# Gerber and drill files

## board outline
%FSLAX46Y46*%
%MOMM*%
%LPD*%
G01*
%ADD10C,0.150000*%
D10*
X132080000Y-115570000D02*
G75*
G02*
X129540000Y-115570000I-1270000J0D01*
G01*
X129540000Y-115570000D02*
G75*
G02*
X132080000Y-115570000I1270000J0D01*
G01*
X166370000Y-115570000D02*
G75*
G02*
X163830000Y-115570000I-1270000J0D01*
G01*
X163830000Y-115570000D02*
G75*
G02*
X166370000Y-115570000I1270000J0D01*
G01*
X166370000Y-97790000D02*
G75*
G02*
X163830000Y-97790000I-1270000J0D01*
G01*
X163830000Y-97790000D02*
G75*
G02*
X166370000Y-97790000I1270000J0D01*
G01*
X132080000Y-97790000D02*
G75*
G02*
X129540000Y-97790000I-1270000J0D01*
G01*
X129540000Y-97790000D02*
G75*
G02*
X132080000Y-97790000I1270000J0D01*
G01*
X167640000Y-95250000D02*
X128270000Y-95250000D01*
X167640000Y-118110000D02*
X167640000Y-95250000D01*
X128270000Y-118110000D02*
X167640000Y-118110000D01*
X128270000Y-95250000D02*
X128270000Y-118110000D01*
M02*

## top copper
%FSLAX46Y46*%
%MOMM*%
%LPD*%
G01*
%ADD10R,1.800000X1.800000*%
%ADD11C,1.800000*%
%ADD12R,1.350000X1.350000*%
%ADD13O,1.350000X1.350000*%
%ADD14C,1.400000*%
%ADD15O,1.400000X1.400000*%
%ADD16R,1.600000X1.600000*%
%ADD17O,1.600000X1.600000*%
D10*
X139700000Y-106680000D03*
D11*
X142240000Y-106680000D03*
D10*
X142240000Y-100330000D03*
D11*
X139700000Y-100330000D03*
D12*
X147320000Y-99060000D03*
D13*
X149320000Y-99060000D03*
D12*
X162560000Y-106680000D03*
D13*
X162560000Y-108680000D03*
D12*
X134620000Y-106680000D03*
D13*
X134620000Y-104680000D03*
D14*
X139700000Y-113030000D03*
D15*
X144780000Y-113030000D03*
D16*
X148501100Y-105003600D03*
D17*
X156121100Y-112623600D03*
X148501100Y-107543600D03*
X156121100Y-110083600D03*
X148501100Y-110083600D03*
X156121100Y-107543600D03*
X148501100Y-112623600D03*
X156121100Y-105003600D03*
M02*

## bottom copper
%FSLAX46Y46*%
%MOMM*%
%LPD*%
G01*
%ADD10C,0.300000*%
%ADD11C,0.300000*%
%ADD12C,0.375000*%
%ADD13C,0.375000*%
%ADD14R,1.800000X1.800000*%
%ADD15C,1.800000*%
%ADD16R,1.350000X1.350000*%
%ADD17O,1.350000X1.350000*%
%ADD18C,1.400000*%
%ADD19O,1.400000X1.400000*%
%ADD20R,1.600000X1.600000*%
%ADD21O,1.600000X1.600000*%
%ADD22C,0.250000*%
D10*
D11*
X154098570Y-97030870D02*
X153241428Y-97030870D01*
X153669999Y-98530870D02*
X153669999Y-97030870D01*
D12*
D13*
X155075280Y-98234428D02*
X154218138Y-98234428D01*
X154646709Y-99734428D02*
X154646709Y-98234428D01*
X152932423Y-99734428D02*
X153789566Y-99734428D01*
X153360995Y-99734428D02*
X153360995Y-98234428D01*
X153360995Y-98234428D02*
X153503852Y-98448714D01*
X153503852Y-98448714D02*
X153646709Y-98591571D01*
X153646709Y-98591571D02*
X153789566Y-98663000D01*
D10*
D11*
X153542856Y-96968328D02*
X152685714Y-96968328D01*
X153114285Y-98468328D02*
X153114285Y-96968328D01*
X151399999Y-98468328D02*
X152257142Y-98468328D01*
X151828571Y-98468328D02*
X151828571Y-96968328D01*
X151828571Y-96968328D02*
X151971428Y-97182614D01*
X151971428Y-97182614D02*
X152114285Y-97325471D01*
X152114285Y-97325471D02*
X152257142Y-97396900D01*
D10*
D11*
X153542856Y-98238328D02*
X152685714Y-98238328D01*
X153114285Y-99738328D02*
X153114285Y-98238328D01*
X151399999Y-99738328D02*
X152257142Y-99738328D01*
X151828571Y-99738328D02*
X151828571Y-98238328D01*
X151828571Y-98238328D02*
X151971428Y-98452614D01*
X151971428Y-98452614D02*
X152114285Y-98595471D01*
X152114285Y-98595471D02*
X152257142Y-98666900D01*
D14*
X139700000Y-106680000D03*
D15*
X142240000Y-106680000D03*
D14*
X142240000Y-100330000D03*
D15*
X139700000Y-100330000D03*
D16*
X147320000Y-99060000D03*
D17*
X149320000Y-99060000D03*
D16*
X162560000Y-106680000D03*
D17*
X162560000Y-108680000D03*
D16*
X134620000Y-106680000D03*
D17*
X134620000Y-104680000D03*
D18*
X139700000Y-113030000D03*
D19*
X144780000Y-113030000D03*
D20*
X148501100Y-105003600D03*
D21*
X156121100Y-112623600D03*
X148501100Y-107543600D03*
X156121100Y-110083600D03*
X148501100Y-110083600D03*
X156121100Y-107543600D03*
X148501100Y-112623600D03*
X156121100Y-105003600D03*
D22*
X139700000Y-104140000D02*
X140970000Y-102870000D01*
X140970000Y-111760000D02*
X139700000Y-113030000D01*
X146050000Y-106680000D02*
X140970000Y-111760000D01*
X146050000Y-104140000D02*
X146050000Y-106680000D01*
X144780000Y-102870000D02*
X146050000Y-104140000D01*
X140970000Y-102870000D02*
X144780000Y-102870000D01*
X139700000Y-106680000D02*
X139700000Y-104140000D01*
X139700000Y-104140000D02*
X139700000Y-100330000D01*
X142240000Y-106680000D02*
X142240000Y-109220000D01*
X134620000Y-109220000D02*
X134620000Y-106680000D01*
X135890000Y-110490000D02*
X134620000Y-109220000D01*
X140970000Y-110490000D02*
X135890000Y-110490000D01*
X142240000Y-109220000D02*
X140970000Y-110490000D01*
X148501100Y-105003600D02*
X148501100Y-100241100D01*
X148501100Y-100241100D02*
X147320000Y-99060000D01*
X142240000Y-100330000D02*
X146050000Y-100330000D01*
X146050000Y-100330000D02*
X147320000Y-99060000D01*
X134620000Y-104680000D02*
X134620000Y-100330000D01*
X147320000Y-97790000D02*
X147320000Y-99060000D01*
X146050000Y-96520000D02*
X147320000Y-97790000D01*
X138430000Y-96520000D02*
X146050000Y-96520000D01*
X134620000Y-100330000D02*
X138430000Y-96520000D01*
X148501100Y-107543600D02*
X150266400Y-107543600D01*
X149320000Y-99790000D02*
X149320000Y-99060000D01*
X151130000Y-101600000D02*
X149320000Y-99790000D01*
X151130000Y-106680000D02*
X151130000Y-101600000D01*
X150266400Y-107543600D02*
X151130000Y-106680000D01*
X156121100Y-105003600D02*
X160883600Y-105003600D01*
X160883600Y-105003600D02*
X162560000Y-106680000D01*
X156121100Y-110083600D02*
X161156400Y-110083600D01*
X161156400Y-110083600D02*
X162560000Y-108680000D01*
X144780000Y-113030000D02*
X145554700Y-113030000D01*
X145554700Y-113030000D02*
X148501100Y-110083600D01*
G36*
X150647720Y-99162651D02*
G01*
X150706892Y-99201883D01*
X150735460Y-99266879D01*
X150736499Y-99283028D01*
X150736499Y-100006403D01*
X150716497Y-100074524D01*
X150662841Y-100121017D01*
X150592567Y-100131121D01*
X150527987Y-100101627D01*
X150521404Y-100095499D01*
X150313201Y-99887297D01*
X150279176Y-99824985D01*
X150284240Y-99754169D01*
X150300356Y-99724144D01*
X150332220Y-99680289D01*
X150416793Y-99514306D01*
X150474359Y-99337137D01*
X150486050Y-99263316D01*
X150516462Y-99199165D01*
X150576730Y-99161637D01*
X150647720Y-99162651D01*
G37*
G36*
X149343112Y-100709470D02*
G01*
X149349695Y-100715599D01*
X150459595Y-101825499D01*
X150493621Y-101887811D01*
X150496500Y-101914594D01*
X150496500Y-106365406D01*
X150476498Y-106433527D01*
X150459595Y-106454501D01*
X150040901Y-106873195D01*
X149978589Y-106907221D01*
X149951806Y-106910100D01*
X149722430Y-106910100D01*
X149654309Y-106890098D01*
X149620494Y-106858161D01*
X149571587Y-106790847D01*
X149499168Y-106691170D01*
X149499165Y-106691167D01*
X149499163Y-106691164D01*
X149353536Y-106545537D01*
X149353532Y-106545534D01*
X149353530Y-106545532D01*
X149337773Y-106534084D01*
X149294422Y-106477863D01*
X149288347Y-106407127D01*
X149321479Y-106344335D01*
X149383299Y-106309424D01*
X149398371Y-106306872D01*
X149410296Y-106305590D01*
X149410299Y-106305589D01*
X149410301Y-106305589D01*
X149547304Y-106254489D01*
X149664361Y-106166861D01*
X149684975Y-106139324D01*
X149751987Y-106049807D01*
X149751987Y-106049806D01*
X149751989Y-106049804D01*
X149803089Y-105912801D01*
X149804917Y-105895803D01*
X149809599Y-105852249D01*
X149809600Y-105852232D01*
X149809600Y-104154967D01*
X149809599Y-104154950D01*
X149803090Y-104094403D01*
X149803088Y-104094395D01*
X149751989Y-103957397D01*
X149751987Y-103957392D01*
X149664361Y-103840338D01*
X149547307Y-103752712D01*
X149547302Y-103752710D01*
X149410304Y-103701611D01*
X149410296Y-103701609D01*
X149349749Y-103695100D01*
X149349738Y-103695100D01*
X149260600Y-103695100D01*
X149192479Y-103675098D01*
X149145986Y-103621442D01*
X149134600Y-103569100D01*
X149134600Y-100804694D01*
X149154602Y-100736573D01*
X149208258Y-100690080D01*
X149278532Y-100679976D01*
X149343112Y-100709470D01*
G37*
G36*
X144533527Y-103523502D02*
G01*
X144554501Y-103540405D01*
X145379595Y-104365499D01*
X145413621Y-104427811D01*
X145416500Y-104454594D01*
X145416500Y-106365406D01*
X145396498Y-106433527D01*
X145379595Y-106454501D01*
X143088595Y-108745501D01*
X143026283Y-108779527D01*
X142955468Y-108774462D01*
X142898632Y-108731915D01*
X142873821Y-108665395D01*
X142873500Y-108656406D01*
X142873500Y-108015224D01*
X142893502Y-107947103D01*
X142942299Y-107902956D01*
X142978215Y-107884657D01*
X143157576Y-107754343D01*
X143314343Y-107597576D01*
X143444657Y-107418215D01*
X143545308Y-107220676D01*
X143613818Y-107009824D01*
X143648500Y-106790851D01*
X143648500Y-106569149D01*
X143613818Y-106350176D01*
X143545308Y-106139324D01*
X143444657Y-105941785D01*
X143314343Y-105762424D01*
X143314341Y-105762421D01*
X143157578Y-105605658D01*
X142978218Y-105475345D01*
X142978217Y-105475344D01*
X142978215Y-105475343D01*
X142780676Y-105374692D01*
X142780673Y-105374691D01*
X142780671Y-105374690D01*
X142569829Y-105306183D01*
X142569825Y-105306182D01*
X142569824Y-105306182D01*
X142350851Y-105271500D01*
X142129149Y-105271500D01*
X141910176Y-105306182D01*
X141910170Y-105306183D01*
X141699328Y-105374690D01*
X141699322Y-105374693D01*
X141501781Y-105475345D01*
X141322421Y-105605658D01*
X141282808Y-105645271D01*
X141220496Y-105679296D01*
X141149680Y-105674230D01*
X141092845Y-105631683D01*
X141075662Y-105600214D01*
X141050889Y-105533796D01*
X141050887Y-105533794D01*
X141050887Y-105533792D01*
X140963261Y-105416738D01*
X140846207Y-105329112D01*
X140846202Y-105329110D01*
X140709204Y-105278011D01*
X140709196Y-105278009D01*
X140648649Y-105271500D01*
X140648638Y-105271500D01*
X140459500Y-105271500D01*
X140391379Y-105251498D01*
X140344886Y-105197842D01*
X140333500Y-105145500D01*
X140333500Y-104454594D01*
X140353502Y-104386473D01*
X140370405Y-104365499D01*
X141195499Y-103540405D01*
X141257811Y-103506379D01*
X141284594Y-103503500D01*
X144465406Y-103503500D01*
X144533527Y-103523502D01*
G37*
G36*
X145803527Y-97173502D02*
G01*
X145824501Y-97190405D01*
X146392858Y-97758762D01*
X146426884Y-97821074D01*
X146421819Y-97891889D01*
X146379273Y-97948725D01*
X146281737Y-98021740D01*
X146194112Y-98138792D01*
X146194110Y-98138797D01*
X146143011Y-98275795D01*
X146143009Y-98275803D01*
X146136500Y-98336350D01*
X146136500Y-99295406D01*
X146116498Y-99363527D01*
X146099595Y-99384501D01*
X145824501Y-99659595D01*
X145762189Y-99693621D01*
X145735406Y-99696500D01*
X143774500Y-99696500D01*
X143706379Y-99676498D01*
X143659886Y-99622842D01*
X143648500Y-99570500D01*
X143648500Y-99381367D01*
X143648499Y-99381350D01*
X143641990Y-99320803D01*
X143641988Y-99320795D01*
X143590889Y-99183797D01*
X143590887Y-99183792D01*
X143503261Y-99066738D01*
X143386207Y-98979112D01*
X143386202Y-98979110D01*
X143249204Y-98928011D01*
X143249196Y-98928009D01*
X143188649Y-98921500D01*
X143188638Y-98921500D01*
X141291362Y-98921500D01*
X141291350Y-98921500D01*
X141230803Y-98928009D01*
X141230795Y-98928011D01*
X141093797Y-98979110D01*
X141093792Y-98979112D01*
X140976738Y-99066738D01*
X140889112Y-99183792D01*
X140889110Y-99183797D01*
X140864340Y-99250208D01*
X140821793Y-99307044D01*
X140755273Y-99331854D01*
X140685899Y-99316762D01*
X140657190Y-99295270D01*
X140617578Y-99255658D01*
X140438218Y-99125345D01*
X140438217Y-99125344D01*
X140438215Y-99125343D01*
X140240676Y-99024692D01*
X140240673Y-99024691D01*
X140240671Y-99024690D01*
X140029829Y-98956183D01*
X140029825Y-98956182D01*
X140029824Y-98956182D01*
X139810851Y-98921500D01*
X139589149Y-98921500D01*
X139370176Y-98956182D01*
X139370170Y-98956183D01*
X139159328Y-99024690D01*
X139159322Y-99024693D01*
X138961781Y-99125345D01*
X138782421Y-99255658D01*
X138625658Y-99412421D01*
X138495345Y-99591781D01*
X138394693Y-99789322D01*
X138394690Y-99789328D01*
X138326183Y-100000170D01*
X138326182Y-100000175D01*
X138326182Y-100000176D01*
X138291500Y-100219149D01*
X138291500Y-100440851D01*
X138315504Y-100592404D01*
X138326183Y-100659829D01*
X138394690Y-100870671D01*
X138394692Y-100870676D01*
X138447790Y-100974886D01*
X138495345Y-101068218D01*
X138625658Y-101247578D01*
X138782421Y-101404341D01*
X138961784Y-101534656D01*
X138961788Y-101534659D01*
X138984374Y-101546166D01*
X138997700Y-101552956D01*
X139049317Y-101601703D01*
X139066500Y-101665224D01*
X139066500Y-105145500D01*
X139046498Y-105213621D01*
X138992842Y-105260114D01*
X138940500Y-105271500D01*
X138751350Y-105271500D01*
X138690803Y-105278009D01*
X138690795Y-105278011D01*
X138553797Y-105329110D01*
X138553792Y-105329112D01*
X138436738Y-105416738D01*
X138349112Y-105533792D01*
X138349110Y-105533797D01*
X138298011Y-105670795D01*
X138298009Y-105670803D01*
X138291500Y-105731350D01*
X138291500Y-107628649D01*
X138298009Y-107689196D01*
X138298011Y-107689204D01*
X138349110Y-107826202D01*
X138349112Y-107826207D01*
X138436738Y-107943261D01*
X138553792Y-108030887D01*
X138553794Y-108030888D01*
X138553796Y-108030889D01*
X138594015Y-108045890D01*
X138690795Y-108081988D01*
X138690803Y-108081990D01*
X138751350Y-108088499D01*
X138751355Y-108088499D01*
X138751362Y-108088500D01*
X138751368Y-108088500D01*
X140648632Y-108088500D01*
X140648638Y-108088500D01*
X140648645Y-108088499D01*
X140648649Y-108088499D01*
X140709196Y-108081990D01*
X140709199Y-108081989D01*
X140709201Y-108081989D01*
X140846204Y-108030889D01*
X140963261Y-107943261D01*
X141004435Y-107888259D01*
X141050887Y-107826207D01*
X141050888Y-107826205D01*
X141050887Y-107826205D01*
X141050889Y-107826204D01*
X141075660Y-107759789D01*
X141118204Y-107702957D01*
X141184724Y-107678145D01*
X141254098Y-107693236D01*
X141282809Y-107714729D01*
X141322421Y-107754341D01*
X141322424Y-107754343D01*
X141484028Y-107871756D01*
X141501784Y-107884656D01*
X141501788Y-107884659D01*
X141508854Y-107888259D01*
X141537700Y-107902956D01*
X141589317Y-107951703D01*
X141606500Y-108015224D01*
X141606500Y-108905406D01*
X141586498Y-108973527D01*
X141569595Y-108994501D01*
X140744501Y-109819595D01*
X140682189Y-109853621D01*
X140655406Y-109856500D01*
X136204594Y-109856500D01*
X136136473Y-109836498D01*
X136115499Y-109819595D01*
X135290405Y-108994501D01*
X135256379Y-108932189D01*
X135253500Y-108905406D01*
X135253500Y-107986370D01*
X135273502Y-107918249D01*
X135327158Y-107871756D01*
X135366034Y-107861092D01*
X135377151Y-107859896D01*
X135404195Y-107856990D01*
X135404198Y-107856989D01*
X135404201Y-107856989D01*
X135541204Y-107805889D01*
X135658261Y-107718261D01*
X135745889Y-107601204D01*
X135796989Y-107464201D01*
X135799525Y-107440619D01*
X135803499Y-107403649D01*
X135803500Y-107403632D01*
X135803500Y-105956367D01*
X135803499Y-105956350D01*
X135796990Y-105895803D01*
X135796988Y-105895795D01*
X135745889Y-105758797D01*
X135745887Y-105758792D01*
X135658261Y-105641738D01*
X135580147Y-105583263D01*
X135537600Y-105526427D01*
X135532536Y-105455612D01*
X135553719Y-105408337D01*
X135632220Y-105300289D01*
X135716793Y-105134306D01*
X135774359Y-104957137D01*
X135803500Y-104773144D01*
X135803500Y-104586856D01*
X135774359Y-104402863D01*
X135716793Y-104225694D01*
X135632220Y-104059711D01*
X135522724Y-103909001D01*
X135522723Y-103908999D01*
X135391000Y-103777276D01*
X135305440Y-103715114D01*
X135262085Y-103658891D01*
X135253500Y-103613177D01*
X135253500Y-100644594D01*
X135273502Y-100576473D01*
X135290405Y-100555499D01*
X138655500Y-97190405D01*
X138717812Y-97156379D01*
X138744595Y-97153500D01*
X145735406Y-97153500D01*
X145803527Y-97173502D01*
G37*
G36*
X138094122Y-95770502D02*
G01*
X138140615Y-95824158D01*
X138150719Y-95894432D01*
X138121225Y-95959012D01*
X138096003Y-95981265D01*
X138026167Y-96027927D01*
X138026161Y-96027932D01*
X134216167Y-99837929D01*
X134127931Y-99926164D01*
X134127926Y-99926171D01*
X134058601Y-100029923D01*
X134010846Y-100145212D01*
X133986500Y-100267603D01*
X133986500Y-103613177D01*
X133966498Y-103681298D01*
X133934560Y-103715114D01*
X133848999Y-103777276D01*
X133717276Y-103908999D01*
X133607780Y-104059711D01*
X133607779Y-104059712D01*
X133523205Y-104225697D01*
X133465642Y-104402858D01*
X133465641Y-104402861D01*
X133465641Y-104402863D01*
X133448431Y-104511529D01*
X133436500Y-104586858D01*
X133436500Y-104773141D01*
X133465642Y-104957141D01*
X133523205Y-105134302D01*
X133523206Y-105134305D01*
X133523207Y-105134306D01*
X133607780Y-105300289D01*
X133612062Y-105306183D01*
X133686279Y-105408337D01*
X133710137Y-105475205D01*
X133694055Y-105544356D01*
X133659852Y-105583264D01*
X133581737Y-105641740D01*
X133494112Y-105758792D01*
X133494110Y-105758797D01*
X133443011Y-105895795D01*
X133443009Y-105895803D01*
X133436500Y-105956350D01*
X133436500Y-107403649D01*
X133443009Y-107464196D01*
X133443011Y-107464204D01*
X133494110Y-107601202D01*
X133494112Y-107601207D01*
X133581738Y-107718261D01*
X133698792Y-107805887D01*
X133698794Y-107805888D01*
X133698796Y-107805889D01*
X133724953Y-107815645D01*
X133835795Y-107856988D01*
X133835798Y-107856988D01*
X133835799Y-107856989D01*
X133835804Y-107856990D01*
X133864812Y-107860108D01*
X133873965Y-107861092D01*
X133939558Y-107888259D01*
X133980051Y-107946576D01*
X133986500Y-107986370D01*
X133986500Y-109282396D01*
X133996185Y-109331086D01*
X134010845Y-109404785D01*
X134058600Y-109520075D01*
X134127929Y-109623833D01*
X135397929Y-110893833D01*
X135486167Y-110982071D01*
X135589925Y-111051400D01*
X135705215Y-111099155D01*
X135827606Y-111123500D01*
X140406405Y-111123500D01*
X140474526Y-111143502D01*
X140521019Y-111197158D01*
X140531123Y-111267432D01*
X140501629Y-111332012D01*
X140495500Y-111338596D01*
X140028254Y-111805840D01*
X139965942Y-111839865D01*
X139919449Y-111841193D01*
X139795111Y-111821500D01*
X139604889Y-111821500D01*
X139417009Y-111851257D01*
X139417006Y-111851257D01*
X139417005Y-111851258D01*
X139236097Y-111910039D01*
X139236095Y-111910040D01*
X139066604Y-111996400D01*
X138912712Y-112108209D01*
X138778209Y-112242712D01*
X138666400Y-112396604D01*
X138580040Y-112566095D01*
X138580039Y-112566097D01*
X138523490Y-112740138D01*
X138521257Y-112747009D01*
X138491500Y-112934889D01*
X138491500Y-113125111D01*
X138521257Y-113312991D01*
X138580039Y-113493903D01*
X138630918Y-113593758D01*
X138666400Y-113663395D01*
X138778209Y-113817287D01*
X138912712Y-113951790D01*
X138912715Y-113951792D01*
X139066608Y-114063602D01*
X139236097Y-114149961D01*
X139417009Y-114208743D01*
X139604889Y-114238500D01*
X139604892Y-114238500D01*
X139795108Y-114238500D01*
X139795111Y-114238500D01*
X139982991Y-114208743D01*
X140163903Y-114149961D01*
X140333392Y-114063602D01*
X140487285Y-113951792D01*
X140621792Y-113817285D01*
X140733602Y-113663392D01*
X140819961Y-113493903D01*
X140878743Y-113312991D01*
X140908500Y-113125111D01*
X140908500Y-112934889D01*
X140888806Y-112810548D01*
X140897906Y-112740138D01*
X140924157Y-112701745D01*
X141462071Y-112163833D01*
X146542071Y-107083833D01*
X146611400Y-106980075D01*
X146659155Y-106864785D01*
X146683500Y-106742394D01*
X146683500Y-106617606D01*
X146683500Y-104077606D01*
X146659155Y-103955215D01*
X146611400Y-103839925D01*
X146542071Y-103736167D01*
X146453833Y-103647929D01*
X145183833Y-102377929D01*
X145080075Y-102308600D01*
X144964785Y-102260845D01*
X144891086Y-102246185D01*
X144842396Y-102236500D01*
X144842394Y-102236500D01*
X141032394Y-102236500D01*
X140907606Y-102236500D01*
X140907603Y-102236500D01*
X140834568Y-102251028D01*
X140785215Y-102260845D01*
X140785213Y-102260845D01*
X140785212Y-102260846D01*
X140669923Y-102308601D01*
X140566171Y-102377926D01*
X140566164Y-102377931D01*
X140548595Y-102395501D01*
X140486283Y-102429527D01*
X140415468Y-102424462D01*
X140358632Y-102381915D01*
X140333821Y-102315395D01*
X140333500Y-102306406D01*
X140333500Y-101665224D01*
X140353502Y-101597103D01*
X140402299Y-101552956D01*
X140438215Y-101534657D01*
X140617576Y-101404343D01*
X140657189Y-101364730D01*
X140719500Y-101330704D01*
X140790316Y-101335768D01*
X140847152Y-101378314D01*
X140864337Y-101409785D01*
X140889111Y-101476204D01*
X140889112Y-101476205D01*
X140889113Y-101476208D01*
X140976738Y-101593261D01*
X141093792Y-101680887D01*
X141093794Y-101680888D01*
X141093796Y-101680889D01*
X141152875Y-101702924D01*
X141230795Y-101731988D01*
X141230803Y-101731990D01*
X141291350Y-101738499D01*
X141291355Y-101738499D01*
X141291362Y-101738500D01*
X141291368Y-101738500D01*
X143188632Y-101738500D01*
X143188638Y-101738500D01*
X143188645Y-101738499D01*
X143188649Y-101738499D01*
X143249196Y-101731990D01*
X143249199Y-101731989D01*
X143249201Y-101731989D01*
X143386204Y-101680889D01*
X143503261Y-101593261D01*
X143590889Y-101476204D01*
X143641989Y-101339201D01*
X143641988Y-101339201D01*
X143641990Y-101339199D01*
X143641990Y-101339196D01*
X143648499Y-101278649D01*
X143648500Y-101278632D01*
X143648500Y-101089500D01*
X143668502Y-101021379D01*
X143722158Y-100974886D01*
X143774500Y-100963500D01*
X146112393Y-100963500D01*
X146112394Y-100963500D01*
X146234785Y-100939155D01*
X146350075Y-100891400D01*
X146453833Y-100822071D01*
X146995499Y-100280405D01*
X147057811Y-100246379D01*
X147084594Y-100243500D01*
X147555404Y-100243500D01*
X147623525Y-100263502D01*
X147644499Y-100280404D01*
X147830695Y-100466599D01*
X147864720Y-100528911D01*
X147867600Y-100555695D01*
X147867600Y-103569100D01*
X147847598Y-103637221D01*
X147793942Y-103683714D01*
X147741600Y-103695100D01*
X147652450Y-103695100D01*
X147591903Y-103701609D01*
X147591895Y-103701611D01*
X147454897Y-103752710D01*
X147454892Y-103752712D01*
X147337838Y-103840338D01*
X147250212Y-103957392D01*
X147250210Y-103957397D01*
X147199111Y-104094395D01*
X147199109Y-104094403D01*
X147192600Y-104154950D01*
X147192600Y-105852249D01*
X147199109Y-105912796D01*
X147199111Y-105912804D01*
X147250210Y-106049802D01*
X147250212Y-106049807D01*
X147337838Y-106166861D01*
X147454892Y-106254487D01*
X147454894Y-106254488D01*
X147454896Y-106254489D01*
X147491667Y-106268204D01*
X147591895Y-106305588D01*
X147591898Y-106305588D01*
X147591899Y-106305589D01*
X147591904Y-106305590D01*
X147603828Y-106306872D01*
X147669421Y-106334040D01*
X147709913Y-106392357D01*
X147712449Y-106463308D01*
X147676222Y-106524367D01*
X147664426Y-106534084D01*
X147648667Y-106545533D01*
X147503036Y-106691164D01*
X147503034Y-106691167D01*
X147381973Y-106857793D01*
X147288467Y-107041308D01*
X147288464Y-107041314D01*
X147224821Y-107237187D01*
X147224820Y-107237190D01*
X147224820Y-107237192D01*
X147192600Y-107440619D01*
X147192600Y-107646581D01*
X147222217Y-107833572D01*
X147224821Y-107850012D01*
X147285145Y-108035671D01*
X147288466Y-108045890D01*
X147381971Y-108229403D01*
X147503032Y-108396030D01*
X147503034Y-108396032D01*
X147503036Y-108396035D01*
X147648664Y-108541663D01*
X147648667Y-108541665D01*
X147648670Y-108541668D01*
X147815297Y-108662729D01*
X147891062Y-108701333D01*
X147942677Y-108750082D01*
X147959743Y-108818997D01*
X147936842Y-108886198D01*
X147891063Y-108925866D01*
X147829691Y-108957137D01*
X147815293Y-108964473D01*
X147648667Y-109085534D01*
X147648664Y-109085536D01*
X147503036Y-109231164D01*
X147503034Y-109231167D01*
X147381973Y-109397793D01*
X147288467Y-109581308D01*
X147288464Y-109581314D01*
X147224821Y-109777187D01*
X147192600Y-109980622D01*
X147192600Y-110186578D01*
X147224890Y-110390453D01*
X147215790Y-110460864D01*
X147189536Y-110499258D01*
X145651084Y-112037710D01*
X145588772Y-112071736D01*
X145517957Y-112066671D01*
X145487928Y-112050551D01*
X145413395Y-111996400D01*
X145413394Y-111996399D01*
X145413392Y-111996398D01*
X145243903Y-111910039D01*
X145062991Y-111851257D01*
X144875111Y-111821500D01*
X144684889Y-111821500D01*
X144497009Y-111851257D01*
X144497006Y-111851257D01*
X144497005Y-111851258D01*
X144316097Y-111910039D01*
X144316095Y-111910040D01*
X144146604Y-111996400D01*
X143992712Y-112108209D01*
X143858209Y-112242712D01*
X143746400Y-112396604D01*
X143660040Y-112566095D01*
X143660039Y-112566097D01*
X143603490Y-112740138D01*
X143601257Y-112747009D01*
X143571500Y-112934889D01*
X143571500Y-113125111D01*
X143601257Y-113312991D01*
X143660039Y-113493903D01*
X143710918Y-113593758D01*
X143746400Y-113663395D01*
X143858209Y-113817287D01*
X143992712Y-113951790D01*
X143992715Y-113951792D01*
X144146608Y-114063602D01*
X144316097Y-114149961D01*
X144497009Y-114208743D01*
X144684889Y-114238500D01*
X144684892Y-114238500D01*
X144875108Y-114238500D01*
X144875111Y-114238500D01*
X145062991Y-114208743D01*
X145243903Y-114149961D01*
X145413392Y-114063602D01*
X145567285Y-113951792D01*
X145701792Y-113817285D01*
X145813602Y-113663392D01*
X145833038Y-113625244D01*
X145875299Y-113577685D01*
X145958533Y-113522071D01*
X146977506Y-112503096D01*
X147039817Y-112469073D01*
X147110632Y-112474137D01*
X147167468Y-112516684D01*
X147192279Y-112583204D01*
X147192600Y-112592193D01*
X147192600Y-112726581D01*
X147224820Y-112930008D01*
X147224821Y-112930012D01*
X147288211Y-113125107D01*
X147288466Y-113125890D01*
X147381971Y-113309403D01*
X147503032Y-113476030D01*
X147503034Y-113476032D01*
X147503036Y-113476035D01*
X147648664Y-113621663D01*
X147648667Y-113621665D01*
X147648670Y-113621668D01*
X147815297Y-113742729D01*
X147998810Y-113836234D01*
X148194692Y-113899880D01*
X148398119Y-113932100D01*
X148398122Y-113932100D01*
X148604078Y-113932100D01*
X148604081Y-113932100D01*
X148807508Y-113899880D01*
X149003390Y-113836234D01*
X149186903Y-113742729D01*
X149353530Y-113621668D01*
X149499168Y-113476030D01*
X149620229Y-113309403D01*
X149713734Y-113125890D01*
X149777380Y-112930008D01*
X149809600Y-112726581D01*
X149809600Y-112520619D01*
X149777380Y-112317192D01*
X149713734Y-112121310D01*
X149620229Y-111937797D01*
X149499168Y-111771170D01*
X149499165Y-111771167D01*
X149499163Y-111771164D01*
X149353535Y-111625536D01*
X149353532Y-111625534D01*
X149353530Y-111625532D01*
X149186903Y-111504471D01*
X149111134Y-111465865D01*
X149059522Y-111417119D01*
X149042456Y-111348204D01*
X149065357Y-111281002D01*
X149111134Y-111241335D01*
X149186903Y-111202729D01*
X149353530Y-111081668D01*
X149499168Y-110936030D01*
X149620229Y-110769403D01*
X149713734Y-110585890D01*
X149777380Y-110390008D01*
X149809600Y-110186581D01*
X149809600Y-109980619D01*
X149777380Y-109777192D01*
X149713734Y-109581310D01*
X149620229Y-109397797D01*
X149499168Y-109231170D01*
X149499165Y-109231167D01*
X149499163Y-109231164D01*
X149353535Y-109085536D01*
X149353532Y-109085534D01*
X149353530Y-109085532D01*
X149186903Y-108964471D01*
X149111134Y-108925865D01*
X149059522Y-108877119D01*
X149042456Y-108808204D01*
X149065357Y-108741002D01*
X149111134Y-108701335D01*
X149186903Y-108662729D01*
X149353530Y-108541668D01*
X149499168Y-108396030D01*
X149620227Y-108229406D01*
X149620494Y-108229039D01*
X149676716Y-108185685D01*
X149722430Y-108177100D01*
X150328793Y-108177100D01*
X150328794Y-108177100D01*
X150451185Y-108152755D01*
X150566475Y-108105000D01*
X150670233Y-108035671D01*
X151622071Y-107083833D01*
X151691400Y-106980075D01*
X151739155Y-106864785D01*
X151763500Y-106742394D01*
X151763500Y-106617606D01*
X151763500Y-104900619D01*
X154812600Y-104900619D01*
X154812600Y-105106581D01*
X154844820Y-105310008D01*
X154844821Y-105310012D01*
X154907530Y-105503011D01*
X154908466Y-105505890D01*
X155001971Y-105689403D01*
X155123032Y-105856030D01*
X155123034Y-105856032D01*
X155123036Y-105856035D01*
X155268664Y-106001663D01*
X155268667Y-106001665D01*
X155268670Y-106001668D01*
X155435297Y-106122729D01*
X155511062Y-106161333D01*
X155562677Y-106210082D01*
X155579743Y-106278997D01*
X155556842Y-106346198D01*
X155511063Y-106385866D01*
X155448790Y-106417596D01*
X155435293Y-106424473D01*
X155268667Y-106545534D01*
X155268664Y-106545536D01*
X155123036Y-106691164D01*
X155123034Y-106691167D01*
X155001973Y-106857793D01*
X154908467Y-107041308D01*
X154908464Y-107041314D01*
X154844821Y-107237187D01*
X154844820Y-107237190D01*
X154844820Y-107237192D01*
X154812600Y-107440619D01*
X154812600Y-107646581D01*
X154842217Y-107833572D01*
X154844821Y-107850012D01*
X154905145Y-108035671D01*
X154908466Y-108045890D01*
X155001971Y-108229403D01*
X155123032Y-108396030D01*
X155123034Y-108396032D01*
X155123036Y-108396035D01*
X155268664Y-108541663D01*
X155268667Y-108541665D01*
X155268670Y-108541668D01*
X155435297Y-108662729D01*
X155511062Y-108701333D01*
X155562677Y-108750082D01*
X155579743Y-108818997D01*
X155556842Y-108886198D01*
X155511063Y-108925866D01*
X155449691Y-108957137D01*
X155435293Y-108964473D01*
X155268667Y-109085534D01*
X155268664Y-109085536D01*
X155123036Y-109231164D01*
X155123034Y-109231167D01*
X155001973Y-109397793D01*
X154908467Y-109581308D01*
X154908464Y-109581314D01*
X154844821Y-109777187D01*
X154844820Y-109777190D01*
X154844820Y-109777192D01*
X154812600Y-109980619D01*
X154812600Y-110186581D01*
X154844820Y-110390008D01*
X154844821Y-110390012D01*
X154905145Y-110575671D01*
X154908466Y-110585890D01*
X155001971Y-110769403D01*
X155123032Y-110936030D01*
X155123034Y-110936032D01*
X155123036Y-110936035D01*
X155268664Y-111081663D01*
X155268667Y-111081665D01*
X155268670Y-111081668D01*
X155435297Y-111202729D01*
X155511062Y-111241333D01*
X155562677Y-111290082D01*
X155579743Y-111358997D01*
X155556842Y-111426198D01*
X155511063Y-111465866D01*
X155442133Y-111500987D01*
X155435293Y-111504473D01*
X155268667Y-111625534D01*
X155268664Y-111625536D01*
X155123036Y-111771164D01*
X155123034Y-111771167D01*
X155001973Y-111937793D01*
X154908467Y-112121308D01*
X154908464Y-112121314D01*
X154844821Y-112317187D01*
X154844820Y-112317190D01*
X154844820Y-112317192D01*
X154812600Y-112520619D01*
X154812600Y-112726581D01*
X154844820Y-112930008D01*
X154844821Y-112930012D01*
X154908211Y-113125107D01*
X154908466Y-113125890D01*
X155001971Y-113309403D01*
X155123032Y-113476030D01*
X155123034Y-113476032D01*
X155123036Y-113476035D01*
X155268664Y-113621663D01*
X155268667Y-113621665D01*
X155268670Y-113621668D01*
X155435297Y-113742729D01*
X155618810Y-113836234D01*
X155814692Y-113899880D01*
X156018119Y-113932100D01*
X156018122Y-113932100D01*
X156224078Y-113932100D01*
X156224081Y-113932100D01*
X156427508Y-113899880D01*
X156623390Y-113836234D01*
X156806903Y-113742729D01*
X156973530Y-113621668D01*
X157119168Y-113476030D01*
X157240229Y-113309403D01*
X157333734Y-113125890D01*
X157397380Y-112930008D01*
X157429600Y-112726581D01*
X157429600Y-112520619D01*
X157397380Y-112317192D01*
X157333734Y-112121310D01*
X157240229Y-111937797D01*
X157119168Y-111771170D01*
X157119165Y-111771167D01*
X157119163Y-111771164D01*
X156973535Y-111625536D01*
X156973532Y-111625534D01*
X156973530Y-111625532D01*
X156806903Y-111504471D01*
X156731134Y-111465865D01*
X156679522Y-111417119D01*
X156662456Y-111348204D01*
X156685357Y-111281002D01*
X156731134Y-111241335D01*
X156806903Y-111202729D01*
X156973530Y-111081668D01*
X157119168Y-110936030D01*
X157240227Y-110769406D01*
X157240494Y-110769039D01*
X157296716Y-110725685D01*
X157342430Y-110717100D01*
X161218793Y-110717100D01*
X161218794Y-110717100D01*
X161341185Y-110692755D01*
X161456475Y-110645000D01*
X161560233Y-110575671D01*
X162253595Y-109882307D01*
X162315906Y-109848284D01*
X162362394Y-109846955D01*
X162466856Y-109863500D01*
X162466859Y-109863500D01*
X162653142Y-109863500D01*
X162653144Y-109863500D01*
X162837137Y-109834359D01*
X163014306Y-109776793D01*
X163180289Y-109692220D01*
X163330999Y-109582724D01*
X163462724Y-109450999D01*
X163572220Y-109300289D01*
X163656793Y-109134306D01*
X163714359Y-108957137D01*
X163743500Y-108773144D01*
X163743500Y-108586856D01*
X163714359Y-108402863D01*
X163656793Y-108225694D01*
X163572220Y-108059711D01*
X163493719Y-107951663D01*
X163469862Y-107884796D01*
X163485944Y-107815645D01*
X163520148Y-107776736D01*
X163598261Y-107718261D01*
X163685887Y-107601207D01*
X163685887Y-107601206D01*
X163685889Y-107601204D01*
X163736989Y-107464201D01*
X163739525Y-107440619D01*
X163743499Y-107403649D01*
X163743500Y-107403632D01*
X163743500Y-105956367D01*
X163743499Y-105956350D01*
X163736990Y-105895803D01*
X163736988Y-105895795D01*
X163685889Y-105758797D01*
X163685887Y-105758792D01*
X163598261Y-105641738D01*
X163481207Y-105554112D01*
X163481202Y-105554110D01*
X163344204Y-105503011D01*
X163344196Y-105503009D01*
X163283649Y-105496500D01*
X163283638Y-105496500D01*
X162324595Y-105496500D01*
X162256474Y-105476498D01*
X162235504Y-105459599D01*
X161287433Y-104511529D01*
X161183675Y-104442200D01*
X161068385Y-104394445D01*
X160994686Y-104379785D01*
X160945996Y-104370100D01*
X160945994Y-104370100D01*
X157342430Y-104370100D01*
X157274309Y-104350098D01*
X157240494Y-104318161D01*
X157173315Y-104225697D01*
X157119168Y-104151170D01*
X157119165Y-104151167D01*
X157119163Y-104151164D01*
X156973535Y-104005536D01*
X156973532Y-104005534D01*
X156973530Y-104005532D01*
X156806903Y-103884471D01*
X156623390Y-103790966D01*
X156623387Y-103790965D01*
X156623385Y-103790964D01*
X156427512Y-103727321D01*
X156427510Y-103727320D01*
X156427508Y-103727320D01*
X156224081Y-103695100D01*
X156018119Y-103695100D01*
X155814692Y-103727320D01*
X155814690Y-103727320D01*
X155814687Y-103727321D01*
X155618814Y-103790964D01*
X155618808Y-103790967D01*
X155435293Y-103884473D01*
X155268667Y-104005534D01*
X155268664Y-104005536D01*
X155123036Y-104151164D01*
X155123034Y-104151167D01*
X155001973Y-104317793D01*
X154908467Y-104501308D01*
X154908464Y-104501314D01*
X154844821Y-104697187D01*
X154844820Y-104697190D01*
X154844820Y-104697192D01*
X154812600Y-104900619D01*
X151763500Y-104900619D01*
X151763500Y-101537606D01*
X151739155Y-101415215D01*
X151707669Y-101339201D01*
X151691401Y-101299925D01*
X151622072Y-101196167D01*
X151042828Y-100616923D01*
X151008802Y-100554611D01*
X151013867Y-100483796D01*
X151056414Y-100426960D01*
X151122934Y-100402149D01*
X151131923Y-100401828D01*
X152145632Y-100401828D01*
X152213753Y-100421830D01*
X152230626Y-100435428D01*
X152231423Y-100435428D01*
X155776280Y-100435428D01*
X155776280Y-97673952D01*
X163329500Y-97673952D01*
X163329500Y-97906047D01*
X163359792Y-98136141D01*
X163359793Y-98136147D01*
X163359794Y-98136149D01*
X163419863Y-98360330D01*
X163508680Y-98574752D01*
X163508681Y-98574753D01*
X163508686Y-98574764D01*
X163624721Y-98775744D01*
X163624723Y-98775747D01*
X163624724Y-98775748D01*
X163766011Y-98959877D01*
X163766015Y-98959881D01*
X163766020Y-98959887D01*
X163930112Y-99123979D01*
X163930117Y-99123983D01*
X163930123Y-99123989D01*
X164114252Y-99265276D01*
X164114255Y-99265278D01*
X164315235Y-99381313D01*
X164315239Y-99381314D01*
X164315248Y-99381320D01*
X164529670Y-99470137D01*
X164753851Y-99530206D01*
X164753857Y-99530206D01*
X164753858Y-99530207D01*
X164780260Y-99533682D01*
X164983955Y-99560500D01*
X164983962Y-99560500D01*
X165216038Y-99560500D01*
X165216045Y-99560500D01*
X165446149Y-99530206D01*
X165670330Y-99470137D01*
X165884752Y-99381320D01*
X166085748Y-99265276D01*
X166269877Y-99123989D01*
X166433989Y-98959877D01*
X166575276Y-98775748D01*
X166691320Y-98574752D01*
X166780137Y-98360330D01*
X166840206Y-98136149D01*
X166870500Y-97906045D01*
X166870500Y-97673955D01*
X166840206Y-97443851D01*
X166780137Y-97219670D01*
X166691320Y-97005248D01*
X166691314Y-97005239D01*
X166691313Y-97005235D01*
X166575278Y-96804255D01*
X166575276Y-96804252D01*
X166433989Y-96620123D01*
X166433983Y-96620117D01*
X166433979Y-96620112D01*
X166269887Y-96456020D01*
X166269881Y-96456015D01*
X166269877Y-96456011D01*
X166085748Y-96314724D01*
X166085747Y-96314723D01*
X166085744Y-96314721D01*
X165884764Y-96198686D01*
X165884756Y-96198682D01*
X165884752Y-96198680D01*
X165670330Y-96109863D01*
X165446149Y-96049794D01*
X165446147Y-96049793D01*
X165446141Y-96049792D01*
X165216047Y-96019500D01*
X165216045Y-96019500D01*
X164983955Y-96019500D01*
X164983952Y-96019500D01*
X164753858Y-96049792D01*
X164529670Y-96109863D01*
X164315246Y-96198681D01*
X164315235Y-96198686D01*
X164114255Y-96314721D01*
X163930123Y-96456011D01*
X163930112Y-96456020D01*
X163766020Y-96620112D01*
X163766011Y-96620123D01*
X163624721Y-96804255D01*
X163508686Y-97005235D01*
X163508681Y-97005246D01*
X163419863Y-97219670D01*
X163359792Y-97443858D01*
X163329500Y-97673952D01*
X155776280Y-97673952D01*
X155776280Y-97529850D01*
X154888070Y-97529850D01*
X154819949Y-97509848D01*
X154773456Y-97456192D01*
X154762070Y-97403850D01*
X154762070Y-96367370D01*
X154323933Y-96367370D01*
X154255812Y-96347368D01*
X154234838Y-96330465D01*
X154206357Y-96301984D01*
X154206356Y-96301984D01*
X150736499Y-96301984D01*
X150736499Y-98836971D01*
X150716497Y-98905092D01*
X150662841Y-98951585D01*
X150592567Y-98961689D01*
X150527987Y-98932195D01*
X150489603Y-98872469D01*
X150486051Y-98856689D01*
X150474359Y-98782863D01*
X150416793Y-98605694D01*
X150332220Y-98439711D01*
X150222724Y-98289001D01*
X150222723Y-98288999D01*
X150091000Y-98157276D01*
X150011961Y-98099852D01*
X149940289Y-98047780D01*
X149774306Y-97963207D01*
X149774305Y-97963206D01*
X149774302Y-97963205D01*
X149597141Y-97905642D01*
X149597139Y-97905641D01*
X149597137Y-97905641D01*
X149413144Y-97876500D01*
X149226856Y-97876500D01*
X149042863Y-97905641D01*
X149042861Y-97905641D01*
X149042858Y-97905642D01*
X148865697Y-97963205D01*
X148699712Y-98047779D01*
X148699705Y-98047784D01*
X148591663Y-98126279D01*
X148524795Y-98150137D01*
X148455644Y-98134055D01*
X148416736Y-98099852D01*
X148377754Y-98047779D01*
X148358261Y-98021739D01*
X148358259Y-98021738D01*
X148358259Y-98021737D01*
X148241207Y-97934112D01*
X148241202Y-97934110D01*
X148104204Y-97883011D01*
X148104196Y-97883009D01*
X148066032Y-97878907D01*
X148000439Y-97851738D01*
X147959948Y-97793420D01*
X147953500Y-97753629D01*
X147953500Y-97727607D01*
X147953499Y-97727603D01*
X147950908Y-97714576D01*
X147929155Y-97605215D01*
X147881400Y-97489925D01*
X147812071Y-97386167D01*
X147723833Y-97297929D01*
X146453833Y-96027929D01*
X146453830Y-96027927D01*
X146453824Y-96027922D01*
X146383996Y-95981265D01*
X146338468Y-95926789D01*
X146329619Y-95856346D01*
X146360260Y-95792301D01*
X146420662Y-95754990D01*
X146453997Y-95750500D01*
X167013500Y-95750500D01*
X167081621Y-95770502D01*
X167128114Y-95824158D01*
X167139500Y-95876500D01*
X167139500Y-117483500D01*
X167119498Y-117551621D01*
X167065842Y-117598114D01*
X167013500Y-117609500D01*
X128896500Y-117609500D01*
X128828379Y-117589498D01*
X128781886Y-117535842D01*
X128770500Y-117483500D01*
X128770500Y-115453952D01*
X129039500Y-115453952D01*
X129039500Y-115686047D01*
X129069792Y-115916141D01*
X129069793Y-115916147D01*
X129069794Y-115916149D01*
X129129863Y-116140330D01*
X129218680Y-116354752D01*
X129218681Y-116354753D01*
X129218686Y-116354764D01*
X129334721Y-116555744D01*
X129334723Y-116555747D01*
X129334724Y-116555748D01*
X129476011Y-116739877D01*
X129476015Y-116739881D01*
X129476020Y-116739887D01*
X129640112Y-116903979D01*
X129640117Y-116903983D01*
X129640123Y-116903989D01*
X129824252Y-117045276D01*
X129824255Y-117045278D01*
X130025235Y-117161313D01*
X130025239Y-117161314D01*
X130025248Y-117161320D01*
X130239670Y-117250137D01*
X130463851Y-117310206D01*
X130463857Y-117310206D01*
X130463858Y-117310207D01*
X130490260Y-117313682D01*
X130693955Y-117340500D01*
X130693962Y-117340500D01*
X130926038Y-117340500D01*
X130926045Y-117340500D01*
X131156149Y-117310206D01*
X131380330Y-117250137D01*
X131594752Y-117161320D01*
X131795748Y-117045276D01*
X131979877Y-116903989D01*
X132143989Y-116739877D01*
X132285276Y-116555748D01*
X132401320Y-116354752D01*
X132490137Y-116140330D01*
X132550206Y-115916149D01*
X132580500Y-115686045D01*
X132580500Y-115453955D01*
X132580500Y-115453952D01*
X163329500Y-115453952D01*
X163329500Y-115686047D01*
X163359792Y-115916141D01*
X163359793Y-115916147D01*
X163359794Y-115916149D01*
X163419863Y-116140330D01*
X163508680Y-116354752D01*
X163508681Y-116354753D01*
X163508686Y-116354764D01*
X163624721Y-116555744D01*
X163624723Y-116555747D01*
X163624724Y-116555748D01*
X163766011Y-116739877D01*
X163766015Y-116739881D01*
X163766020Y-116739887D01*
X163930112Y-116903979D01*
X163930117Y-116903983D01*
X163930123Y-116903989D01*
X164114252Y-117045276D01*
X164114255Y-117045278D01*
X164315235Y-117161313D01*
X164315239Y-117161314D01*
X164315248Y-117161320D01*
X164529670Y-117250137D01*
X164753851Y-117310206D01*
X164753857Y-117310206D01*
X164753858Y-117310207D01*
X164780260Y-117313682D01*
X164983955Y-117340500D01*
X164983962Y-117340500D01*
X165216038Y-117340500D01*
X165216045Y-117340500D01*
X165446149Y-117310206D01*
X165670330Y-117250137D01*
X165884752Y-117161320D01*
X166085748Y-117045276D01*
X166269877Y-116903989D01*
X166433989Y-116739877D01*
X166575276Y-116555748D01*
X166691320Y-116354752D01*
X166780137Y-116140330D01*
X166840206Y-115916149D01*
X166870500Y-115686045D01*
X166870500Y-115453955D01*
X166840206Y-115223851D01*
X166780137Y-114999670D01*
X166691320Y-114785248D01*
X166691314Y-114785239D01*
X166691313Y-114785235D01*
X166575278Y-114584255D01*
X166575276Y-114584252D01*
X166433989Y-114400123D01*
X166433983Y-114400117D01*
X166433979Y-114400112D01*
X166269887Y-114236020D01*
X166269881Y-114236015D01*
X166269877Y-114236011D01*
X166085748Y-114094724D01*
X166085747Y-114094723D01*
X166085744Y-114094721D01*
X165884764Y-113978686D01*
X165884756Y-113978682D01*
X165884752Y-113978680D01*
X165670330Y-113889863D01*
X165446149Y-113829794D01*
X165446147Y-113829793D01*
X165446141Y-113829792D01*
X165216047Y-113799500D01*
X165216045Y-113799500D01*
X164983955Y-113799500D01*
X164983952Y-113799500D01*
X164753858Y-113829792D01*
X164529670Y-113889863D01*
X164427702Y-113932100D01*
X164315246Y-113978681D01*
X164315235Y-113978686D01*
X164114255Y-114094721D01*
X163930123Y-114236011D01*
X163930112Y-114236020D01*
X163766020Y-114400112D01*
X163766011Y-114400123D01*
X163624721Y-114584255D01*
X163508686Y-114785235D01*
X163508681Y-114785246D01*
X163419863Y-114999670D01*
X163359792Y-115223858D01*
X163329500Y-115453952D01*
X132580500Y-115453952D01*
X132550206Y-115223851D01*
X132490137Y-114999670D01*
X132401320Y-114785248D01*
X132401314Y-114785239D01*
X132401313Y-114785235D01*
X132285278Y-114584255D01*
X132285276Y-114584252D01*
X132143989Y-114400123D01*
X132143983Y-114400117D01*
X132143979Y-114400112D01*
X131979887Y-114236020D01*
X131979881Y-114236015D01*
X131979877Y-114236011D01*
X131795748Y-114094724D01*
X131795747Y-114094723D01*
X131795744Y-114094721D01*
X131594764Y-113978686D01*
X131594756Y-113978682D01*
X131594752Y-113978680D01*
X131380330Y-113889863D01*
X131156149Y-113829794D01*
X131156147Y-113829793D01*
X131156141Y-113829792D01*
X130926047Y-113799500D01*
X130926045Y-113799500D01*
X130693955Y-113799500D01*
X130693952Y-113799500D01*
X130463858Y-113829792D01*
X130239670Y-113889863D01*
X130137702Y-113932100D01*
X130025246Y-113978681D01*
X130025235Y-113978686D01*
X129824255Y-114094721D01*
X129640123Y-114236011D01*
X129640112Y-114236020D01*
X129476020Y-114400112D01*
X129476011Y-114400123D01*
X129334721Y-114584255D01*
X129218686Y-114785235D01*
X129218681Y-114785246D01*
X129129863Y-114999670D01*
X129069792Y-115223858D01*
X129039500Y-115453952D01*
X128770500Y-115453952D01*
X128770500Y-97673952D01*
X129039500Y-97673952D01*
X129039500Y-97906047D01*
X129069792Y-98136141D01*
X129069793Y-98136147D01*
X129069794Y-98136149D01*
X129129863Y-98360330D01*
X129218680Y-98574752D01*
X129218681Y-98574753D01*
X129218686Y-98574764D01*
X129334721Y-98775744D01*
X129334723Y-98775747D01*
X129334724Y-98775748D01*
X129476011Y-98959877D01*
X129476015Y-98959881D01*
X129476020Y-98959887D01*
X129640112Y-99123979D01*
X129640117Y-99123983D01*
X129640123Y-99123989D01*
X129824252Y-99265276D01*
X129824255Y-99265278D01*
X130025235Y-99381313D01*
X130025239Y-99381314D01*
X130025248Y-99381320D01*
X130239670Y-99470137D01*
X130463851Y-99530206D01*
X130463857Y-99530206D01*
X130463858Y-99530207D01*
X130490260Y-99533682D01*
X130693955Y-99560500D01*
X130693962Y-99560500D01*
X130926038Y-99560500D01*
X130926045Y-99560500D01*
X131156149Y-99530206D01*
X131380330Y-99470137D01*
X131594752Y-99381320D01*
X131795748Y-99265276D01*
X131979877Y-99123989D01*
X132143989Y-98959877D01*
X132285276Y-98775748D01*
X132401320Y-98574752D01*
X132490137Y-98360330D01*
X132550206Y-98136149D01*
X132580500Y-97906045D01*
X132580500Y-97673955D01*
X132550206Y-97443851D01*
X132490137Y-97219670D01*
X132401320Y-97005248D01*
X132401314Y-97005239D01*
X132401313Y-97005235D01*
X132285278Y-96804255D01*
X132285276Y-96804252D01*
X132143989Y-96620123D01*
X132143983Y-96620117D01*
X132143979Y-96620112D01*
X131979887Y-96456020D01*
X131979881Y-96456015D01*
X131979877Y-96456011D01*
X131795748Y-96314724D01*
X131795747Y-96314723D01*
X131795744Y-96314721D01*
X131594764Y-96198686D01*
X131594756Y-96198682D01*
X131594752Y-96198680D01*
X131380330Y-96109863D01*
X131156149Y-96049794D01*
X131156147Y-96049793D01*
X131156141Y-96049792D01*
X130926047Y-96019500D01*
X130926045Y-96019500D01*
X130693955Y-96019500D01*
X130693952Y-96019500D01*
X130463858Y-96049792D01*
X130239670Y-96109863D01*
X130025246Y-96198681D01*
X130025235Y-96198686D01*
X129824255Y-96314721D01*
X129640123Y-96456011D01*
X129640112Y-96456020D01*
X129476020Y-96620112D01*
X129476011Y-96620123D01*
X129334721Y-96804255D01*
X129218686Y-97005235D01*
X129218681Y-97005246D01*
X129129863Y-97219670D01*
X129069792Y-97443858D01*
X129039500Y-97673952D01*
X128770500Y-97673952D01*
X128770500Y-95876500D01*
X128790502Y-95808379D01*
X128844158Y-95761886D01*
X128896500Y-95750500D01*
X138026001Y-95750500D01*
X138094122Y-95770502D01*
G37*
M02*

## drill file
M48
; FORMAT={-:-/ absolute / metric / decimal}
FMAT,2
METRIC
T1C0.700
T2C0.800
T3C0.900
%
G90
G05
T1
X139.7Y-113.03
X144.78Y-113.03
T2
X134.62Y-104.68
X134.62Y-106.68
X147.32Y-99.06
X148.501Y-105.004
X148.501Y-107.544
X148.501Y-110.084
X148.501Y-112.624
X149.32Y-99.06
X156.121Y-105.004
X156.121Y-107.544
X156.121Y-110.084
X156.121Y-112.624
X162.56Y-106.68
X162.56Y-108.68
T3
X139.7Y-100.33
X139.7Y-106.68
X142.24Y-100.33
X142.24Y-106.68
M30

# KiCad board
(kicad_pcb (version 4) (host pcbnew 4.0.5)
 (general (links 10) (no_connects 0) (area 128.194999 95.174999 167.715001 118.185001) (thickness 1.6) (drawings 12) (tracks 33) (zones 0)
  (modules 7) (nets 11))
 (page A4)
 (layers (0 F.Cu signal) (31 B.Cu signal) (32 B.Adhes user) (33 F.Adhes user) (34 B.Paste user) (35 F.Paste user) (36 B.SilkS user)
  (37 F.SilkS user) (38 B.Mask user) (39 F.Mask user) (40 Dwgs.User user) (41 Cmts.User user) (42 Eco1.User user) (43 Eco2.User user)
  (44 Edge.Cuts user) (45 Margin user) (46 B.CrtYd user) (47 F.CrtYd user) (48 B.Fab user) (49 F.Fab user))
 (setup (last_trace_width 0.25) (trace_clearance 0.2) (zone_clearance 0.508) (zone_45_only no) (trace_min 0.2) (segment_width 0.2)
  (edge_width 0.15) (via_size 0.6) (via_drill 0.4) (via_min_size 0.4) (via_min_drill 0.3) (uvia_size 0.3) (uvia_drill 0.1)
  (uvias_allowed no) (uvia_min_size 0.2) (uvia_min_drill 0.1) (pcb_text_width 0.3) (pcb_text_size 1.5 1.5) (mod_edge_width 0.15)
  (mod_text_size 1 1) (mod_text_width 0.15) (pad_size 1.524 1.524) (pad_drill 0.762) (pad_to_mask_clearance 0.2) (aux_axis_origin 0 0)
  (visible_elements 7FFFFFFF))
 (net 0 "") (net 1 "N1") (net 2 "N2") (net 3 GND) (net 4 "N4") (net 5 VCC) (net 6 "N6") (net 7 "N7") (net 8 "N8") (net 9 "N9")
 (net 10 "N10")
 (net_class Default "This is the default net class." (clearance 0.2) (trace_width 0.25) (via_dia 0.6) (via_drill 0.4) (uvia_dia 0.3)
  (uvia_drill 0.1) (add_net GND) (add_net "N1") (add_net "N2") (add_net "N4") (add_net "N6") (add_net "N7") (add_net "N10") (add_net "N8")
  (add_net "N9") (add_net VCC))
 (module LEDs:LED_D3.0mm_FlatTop (layer F.Cu) (at 139.7 106.68)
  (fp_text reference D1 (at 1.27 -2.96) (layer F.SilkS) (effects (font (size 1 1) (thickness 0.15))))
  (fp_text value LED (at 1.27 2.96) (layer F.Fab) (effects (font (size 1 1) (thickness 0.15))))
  (pad 1 thru_hole rect (at 0 0) (size 1.8 1.8) (drill 0.9) (layers *.Cu *.Mask) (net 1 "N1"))
  (pad 2 thru_hole circle (at 2.54 0) (size 1.8 1.8) (drill 0.9) (layers *.Cu *.Mask) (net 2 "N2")))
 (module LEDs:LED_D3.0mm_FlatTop (layer F.Cu) (at 142.24 100.33 180)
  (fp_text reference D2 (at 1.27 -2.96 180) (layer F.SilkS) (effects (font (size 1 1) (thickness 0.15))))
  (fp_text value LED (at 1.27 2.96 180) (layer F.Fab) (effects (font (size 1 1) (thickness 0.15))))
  (pad 1 thru_hole rect (at 0 0 180) (size 1.8 1.8) (drill 0.9) (layers *.Cu *.Mask) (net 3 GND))
  (pad 2 thru_hole circle (at 2.54 0 180) (size 1.8 1.8) (drill 0.9) (layers *.Cu *.Mask) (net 1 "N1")))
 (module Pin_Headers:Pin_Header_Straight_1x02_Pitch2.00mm (layer F.Cu) (at 147.32 99.06 90)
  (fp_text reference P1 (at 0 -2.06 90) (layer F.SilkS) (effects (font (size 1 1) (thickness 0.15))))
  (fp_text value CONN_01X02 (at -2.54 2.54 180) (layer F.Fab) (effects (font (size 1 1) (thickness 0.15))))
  (pad 1 thru_hole rect (at 0 0 90) (size 1.35 1.35) (drill 0.8) (layers *.Cu *.Mask) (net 3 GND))
  (pad 2 thru_hole oval (at 0 2 90) (size 1.35 1.35) (drill 0.8) (layers *.Cu *.Mask) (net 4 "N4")))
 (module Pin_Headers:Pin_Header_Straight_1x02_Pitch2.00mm (layer F.Cu) (at 162.56 106.68)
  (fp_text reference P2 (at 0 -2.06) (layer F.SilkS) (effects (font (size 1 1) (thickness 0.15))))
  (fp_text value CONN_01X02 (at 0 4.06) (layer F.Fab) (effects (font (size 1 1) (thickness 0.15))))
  (pad 1 thru_hole rect (at 0 0) (size 1.35 1.35) (drill 0.8) (layers *.Cu *.Mask) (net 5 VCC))
  (pad 2 thru_hole oval (at 0 2) (size 1.35 1.35) (drill 0.8) (layers *.Cu *.Mask) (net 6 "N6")))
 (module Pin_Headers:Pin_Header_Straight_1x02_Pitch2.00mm (layer F.Cu) (at 134.62 106.68 180)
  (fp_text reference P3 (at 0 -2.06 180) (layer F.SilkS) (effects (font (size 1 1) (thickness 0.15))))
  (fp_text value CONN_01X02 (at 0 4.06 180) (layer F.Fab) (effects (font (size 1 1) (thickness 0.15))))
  (pad 1 thru_hole rect (at 0 0 180) (size 1.35 1.35) (drill 0.8) (layers *.Cu *.Mask) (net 2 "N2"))
  (pad 2 thru_hole oval (at 0 2 180) (size 1.35 1.35) (drill 0.8) (layers *.Cu *.Mask) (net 3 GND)))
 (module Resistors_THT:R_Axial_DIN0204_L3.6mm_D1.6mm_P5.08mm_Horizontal (layer F.Cu) (at 139.7 113.03)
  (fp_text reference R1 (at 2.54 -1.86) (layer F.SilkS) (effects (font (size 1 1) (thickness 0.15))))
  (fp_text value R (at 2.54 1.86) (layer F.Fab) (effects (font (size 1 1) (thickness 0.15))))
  (pad 1 thru_hole circle (at 0 0) (size 1.4 1.4) (drill 0.7) (layers *.Cu *.Mask) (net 1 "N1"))
  (pad 2 thru_hole oval (at 5.08 0) (size 1.4 1.4) (drill 0.7) (layers *.Cu *.Mask) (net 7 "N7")))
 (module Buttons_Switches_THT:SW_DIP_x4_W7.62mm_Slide (layer F.Cu) (at 148.5011 105.0036)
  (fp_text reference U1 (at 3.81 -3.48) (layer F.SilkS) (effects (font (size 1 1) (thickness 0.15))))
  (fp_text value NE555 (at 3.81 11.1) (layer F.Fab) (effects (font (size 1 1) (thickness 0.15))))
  (pad 1 thru_hole rect (at 0 0) (size 1.6 1.6) (drill 0.8) (layers *.Cu *.Mask) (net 3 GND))
  (pad 5 thru_hole oval (at 7.62 7.62) (size 1.6 1.6) (drill 0.8) (layers *.Cu *.Mask) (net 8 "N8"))
  (pad 2 thru_hole oval (at 0 2.54) (size 1.6 1.6) (drill 0.8) (layers *.Cu *.Mask) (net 4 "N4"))
  (pad 6 thru_hole oval (at 7.62 5.08) (size 1.6 1.6) (drill 0.8) (layers *.Cu *.Mask) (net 6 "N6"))
  (pad 3 thru_hole oval (at 0 5.08) (size 1.6 1.6) (drill 0.8) (layers *.Cu *.Mask) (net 7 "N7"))
  (pad 7 thru_hole oval (at 7.62 2.54) (size 1.6 1.6) (drill 0.8) (layers *.Cu *.Mask) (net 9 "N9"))
  (pad 4 thru_hole oval (at 0 7.62) (size 1.6 1.6) (drill 0.8) (layers *.Cu *.Mask) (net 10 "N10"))
  (pad 8 thru_hole oval (at 7.62 0) (size 1.6 1.6) (drill 0.8) (layers *.Cu *.Mask) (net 5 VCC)))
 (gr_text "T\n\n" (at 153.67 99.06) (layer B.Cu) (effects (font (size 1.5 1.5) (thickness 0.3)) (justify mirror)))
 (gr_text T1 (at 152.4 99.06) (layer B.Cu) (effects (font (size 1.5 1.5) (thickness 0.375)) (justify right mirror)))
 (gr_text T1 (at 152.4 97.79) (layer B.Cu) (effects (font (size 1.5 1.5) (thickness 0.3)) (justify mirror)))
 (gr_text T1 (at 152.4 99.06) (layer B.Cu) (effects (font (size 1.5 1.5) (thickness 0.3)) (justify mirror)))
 (gr_circle (center 130.81 115.57) (end 130.81 114.3) (layer Edge.Cuts) (width 0.15))
 (gr_circle (center 165.1 115.57) (end 165.1 114.3) (layer Edge.Cuts) (width 0.15))
 (gr_circle (center 165.1 97.79) (end 165.1 96.52) (layer Edge.Cuts) (width 0.15))
 (gr_circle (center 130.81 97.79) (end 130.81 96.52) (layer Edge.Cuts) (width 0.15))
 (gr_line (start 167.64 95.25) (end 128.27 95.25) (angle 90) (layer Edge.Cuts) (width 0.15))
 (gr_line (start 167.64 118.11) (end 167.64 95.25) (angle 90) (layer Edge.Cuts) (width 0.15))
 (gr_line (start 128.27 118.11) (end 167.64 118.11) (angle 90) (layer Edge.Cuts) (width 0.15))
 (gr_line (start 128.27 95.25) (end 128.27 118.11) (angle 90) (layer Edge.Cuts) (width 0.15))
 (segment (start 139.7 104.14) (end 140.97 102.87) (width 0.25) (layer B.Cu) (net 1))
 (segment (start 140.97 111.76) (end 139.7 113.03) (width 0.25) (layer B.Cu) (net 1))
 (segment (start 146.05 106.68) (end 140.97 111.76) (width 0.25) (layer B.Cu) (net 1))
 (segment (start 146.05 104.14) (end 146.05 106.68) (width 0.25) (layer B.Cu) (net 1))
 (segment (start 144.78 102.87) (end 146.05 104.14) (width 0.25) (layer B.Cu) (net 1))
 (segment (start 140.97 102.87) (end 144.78 102.87) (width 0.25) (layer B.Cu) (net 1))
 (segment (start 139.7 106.68) (end 139.7 104.14) (width 0.25) (layer B.Cu) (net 1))
 (segment (start 139.7 104.14) (end 139.7 100.33) (width 0.25) (layer B.Cu) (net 1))
 (segment (start 142.24 106.68) (end 142.24 109.22) (width 0.25) (layer B.Cu) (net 2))
 (segment (start 134.62 109.22) (end 134.62 106.68) (width 0.25) (layer B.Cu) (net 2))
 (segment (start 135.89 110.49) (end 134.62 109.22) (width 0.25) (layer B.Cu) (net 2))
 (segment (start 140.97 110.49) (end 135.89 110.49) (width 0.25) (layer B.Cu) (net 2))
 (segment (start 142.24 109.22) (end 140.97 110.49) (width 0.25) (layer B.Cu) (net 2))
 (segment (start 148.5011 105.0036) (end 148.5011 100.2411) (width 0.25) (layer B.Cu) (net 3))
 (segment (start 148.5011 100.2411) (end 147.32 99.06) (width 0.25) (layer B.Cu) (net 3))
 (segment (start 142.24 100.33) (end 146.05 100.33) (width 0.25) (layer B.Cu) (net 3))
 (segment (start 146.05 100.33) (end 147.32 99.06) (width 0.25) (layer B.Cu) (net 3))
 (segment (start 134.62 104.68) (end 134.62 100.33) (width 0.25) (layer B.Cu) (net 3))
 (segment (start 147.32 97.79) (end 147.32 99.06) (width 0.25) (layer B.Cu) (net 3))
 (segment (start 146.05 96.52) (end 147.32 97.79) (width 0.25) (layer B.Cu) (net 3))
 (segment (start 138.43 96.52) (end 146.05 96.52) (width 0.25) (layer B.Cu) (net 3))
 (segment (start 134.62 100.33) (end 138.43 96.52) (width 0.25) (layer B.Cu) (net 3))
 (segment (start 148.5011 107.5436) (end 150.2664 107.5436) (width 0.25) (layer B.Cu) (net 4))
 (segment (start 149.32 99.79) (end 149.32 99.06) (width 0.25) (layer B.Cu) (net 4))
 (segment (start 151.13 101.6) (end 149.32 99.79) (width 0.25) (layer B.Cu) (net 4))
 (segment (start 151.13 106.68) (end 151.13 101.6) (width 0.25) (layer B.Cu) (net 4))
 (segment (start 150.2664 107.5436) (end 151.13 106.68) (width 0.25) (layer B.Cu) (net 4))
 (segment (start 156.1211 105.0036) (end 160.8836 105.0036) (width 0.25) (layer B.Cu) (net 5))
 (segment (start 160.8836 105.0036) (end 162.56 106.68) (width 0.25) (layer B.Cu) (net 5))
 (segment (start 156.1211 110.0836) (end 161.1564 110.0836) (width 0.25) (layer B.Cu) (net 6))
 (segment (start 161.1564 110.0836) (end 162.56 108.68) (width 0.25) (layer B.Cu) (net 6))
 (segment (start 144.78 113.03) (end 145.5547 113.03) (width 0.25) (layer B.Cu) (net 7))
 (segment (start 145.5547 113.03) (end 148.5011 110.0836) (width 0.25) (layer B.Cu) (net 7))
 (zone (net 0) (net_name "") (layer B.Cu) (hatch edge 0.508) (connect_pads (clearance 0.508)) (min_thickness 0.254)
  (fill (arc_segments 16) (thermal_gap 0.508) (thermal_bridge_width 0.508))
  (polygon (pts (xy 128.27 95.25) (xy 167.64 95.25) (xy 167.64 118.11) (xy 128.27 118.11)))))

